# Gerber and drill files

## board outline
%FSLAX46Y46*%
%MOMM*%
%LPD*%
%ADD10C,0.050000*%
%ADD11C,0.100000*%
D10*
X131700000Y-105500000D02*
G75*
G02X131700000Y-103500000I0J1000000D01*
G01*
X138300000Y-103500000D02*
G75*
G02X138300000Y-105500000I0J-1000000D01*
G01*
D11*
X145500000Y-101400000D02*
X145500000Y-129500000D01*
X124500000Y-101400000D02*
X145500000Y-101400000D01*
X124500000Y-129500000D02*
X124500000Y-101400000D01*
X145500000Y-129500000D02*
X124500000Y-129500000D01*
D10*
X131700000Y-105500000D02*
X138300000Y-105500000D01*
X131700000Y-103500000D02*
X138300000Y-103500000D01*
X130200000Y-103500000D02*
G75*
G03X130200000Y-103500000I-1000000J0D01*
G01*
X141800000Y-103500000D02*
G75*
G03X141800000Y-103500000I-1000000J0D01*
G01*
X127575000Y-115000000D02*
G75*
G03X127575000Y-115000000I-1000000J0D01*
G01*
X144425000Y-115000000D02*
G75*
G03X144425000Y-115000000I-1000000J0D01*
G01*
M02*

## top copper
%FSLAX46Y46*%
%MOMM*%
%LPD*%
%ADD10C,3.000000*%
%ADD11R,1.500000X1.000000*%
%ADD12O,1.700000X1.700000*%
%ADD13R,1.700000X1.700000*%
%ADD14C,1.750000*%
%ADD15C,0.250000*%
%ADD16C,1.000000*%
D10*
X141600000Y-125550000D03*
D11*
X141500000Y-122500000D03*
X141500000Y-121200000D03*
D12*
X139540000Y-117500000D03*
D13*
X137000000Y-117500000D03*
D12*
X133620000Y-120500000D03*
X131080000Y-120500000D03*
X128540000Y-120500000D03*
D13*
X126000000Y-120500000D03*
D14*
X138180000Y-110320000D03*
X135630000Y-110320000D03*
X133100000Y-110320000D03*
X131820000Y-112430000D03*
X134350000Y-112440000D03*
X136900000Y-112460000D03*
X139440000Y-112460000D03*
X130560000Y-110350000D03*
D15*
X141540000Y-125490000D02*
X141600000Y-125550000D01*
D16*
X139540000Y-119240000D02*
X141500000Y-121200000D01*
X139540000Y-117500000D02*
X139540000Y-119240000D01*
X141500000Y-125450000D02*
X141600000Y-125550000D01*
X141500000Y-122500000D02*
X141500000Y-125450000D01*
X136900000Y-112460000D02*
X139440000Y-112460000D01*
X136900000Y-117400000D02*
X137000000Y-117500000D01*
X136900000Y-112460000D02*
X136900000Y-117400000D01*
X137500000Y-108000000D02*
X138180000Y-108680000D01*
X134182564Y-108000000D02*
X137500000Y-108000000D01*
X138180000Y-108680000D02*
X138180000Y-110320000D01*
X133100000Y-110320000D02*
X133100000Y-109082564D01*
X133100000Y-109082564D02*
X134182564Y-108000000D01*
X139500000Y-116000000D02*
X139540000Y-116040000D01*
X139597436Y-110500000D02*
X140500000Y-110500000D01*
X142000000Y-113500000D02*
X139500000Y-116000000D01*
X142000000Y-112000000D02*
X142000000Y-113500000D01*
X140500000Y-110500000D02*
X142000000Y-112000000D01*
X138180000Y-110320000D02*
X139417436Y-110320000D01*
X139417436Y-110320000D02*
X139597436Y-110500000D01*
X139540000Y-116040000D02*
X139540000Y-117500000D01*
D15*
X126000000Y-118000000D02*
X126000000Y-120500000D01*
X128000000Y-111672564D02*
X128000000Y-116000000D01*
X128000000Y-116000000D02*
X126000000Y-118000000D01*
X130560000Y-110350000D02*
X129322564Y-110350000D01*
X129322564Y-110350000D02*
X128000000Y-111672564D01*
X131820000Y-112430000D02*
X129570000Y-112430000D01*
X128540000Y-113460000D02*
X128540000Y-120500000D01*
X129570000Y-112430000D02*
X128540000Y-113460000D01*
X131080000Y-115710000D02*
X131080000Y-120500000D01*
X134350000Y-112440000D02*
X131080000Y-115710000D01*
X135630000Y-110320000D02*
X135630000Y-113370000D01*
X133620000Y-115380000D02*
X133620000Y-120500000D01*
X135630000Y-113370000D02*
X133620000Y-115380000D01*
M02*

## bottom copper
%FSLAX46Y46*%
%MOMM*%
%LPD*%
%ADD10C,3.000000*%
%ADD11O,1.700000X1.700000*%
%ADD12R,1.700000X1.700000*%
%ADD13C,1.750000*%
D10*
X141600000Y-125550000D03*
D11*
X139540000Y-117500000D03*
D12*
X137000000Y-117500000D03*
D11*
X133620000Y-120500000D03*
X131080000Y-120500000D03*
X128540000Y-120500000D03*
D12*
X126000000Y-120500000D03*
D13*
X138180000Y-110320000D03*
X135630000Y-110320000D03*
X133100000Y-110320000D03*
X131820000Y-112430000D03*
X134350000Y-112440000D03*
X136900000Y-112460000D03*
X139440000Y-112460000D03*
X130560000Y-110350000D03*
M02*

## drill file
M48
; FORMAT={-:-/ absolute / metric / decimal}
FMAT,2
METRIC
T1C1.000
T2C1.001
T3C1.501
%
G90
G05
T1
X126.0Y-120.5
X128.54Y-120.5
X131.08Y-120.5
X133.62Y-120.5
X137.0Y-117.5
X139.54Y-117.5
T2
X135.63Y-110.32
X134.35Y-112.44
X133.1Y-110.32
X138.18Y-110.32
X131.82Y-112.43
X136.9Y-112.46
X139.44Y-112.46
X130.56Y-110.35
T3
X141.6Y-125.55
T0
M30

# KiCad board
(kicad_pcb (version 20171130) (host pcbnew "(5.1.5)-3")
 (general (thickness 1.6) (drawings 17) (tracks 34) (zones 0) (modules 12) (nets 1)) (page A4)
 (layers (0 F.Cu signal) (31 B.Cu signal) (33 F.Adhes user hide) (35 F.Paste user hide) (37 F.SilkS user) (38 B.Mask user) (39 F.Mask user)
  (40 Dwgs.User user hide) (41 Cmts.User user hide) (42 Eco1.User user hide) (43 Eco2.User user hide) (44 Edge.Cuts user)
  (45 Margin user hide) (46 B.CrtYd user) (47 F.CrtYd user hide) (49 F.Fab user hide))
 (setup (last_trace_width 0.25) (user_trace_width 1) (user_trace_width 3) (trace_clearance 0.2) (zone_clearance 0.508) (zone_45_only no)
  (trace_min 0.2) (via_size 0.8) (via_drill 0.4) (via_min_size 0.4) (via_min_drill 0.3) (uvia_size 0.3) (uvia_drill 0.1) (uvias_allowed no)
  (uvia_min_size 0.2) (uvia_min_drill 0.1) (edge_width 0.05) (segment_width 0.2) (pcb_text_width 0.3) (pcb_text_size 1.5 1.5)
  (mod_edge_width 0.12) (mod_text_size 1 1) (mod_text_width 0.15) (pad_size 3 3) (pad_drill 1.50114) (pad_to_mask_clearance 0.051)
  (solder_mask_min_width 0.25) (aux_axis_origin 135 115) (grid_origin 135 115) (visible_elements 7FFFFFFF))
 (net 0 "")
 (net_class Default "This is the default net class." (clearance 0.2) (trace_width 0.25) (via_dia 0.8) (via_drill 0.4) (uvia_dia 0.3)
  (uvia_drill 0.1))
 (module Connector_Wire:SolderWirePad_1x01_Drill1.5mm (layer F.Cu) (at 141.6 125.55)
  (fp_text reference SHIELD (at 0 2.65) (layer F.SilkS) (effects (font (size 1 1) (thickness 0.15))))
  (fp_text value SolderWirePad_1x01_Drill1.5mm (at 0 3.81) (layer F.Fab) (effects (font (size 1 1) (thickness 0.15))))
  (pad 1 thru_hole circle (at 0 0) (size 3 3) (drill 1.50114) (layers *.Cu *.Mask)))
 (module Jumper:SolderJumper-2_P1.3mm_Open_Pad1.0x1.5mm (layer F.Cu) (at 141.5 121.85 90)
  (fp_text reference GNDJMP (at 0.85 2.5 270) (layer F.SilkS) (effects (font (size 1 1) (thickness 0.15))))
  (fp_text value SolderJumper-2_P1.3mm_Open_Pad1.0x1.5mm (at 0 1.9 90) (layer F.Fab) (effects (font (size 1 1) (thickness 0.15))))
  (pad 1 smd rect (at -0.65 0 90) (size 1 1.5) (layers F.Cu F.Mask))
  (pad 2 smd rect (at 0.65 0 90) (size 1 1.5) (layers F.Cu F.Mask)))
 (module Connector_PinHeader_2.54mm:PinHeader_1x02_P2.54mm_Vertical (layer F.Cu) (at 137 117.5 90)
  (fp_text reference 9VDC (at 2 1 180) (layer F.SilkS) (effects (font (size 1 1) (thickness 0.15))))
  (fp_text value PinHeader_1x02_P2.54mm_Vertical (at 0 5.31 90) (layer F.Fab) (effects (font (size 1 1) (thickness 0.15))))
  (pad 2 thru_hole oval (at 0 2.54 90) (size 1.7 1.7) (drill 1) (layers *.Cu *.Mask))
  (pad 1 thru_hole rect (at 0 0 90) (size 1.7 1.7) (drill 1) (layers *.Cu *.Mask)))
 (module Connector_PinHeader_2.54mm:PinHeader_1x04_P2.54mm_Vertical (layer F.Cu) (at 126 120.5 90)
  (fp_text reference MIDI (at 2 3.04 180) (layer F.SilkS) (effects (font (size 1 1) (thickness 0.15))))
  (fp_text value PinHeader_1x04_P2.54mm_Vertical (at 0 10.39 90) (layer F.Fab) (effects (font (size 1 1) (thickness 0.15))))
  (pad 4 thru_hole oval (at 0 7.62 90) (size 1.7 1.7) (drill 1) (layers *.Cu *.Mask))
  (pad 3 thru_hole oval (at 0 5.08 90) (size 1.7 1.7) (drill 1) (layers *.Cu *.Mask))
  (pad 2 thru_hole oval (at 0 2.54 90) (size 1.7 1.7) (drill 1) (layers *.Cu *.Mask))
  (pad 1 thru_hole rect (at 0 0 90) (size 1.7 1.7) (drill 1) (layers *.Cu *.Mask)))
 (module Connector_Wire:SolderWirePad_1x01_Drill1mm (layer F.Cu) (at 138.18 110.32)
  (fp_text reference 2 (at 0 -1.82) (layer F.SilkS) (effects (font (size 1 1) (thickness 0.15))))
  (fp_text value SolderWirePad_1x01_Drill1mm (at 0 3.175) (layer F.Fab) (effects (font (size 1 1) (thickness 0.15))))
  (pad 1 thru_hole circle (at 0 0) (size 1.75 1.75) (drill 1.00076) (layers *.Cu *.Mask)))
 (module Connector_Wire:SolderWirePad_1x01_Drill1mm (layer F.Cu) (at 135.63 110.32)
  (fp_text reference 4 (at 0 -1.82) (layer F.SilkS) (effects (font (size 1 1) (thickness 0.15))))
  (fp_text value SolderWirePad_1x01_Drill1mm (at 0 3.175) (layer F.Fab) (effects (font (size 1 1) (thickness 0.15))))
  (pad 1 thru_hole circle (at 0 0) (size 1.75 1.75) (drill 1.00076) (layers *.Cu *.Mask)))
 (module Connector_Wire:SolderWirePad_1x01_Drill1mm (layer F.Cu) (at 133.1 110.32)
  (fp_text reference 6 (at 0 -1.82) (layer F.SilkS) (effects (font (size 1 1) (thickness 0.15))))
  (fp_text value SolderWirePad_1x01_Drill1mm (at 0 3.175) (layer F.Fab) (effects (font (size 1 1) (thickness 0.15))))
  (pad 1 thru_hole circle (at 0 0) (size 1.75 1.75) (drill 1.00076) (layers *.Cu *.Mask)))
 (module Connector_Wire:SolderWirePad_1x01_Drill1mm (layer F.Cu) (at 131.82 112.43)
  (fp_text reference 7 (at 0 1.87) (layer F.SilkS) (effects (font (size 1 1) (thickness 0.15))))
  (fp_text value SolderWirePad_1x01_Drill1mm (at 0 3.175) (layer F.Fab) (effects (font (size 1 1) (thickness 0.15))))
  (pad 1 thru_hole circle (at 0 0) (size 1.75 1.75) (drill 1.00076) (layers *.Cu *.Mask)))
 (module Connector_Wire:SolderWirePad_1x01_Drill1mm (layer F.Cu) (at 134.35 112.44)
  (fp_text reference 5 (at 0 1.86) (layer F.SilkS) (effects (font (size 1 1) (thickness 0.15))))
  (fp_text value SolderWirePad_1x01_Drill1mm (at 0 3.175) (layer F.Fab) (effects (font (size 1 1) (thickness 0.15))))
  (pad 1 thru_hole circle (at 0 0) (size 1.75 1.75) (drill 1.00076) (layers *.Cu *.Mask)))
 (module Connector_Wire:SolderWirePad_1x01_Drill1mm (layer F.Cu) (at 136.9 112.46)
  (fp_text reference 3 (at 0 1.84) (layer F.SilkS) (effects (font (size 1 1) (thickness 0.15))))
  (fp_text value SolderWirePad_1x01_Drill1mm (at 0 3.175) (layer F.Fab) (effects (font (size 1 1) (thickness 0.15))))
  (pad 1 thru_hole circle (at 0 0) (size 1.75 1.75) (drill 1.00076) (layers *.Cu *.Mask)))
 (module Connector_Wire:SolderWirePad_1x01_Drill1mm (layer F.Cu) (at 139.44 112.46)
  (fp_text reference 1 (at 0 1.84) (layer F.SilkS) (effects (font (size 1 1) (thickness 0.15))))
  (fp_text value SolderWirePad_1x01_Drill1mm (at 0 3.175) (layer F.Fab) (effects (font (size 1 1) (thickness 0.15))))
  (pad 1 thru_hole circle (at 0 0) (size 1.75 1.75) (drill 1.00076) (layers *.Cu *.Mask)))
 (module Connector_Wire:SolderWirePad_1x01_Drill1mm (layer F.Cu) (at 130.56 110.35)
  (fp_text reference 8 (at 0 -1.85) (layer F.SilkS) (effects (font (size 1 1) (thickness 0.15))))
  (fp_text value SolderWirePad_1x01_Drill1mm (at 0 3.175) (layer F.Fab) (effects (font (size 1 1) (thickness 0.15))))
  (pad 1 thru_hole circle (at 0 0) (size 1.75 1.75) (drill 1.00076) (layers *.Cu *.Mask)))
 (gr_arc (start 131.7 104.5) (end 131.7 103.5) (angle -180) (layer Edge.Cuts) (width 0.05))
 (gr_arc (start 138.3 104.5) (end 138.3 105.5) (angle -180) (layer Edge.Cuts) (width 0.05))
 (gr_line (start 145.5 101.4) (end 145.5 129.5) (layer Edge.Cuts) (width 0.1))
 (gr_line (start 124.5 101.4) (end 145.5 101.4) (layer Edge.Cuts) (width 0.1))
 (gr_line (start 124.5 129.5) (end 124.5 101.4) (layer Edge.Cuts) (width 0.1))
 (gr_line (start 145.5 129.5) (end 124.5 129.5) (layer Edge.Cuts) (width 0.1))
 (gr_line (start 131.7 105.5) (end 138.3 105.5) (layer Edge.Cuts) (width 0.05))
 (gr_line (start 131.7 103.5) (end 138.3 103.5) (layer Edge.Cuts) (width 0.05))
 (gr_circle (center 129.2 103.5) (end 130.2 103.5) (layer Edge.Cuts) (width 0.05))
 (gr_circle (center 140.8 103.5) (end 141.8 103.5) (layer Edge.Cuts) (width 0.05))
 (gr_circle (center 126.575 115) (end 127.575 115) (layer Edge.Cuts) (width 0.05))
 (gr_circle (center 143.425 115) (end 144.425 115) (layer Edge.Cuts) (width 0.05))
 (segment (start 141.54 125.49) (end 141.6 125.55) (width 0.25) (layer F.Cu) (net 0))
 (segment (start 139.54 119.24) (end 141.5 121.2) (width 1) (layer F.Cu) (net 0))
 (segment (start 139.54 117.5) (end 139.54 119.24) (width 1) (layer F.Cu) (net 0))
 (segment (start 141.5 125.45) (end 141.6 125.55) (width 1) (layer F.Cu) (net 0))
 (segment (start 141.5 122.5) (end 141.5 125.45) (width 1) (layer F.Cu) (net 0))
 (segment (start 136.9 112.46) (end 139.44 112.46) (width 1) (layer F.Cu) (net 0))
 (segment (start 136.9 117.4) (end 137 117.5) (width 1) (layer F.Cu) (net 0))
 (segment (start 136.9 112.46) (end 136.9 117.4) (width 1) (layer F.Cu) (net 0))
 (segment (start 137.5 108) (end 138.18 108.68) (width 1) (layer F.Cu) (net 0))
 (segment (start 134.182564 108) (end 137.5 108) (width 1) (layer F.Cu) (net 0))
 (segment (start 138.18 108.68) (end 138.18 110.32) (width 1) (layer F.Cu) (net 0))
 (segment (start 133.1 110.32) (end 133.1 109.082564) (width 1) (layer F.Cu) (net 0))
 (segment (start 133.1 109.082564) (end 134.182564 108) (width 1) (layer F.Cu) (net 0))
 (segment (start 139.5 116) (end 139.54 116.04) (width 1) (layer F.Cu) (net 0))
 (segment (start 139.597436 110.5) (end 140.5 110.5) (width 1) (layer F.Cu) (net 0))
 (segment (start 142 113.5) (end 139.5 116) (width 1) (layer F.Cu) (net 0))
 (segment (start 142 112) (end 142 113.5) (width 1) (layer F.Cu) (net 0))
 (segment (start 140.5 110.5) (end 142 112) (width 1) (layer F.Cu) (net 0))
 (segment (start 138.18 110.32) (end 139.417436 110.32) (width 1) (layer F.Cu) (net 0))
 (segment (start 139.417436 110.32) (end 139.597436 110.5) (width 1) (layer F.Cu) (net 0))
 (segment (start 139.54 116.04) (end 139.54 117.5) (width 1) (layer F.Cu) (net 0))
 (segment (start 126 118) (end 126 120.5) (width 0.25) (layer F.Cu) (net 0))
 (segment (start 128 111.672564) (end 128 116) (width 0.25) (layer F.Cu) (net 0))
 (segment (start 128 116) (end 126 118) (width 0.25) (layer F.Cu) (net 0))
 (segment (start 130.56 110.35) (end 129.322564 110.35) (width 0.25) (layer F.Cu) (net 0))
 (segment (start 129.322564 110.35) (end 128 111.672564) (width 0.25) (layer F.Cu) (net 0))
 (segment (start 131.82 112.43) (end 129.57 112.43) (width 0.25) (layer F.Cu) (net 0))
 (segment (start 128.54 113.46) (end 128.54 120.5) (width 0.25) (layer F.Cu) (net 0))
 (segment (start 129.57 112.43) (end 128.54 113.46) (width 0.25) (layer F.Cu) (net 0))
 (segment (start 131.08 115.71) (end 131.08 120.5) (width 0.25) (layer F.Cu) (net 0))
 (segment (start 134.35 112.44) (end 131.08 115.71) (width 0.25) (layer F.Cu) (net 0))
 (segment (start 135.63 110.32) (end 135.63 113.37) (width 0.25) (layer F.Cu) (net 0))
 (segment (start 133.62 115.38) (end 133.62 120.5) (width 0.25) (layer F.Cu) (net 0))
 (segment (start 135.63 113.37) (end 133.62 115.38) (width 0.25) (layer F.Cu) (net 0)))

